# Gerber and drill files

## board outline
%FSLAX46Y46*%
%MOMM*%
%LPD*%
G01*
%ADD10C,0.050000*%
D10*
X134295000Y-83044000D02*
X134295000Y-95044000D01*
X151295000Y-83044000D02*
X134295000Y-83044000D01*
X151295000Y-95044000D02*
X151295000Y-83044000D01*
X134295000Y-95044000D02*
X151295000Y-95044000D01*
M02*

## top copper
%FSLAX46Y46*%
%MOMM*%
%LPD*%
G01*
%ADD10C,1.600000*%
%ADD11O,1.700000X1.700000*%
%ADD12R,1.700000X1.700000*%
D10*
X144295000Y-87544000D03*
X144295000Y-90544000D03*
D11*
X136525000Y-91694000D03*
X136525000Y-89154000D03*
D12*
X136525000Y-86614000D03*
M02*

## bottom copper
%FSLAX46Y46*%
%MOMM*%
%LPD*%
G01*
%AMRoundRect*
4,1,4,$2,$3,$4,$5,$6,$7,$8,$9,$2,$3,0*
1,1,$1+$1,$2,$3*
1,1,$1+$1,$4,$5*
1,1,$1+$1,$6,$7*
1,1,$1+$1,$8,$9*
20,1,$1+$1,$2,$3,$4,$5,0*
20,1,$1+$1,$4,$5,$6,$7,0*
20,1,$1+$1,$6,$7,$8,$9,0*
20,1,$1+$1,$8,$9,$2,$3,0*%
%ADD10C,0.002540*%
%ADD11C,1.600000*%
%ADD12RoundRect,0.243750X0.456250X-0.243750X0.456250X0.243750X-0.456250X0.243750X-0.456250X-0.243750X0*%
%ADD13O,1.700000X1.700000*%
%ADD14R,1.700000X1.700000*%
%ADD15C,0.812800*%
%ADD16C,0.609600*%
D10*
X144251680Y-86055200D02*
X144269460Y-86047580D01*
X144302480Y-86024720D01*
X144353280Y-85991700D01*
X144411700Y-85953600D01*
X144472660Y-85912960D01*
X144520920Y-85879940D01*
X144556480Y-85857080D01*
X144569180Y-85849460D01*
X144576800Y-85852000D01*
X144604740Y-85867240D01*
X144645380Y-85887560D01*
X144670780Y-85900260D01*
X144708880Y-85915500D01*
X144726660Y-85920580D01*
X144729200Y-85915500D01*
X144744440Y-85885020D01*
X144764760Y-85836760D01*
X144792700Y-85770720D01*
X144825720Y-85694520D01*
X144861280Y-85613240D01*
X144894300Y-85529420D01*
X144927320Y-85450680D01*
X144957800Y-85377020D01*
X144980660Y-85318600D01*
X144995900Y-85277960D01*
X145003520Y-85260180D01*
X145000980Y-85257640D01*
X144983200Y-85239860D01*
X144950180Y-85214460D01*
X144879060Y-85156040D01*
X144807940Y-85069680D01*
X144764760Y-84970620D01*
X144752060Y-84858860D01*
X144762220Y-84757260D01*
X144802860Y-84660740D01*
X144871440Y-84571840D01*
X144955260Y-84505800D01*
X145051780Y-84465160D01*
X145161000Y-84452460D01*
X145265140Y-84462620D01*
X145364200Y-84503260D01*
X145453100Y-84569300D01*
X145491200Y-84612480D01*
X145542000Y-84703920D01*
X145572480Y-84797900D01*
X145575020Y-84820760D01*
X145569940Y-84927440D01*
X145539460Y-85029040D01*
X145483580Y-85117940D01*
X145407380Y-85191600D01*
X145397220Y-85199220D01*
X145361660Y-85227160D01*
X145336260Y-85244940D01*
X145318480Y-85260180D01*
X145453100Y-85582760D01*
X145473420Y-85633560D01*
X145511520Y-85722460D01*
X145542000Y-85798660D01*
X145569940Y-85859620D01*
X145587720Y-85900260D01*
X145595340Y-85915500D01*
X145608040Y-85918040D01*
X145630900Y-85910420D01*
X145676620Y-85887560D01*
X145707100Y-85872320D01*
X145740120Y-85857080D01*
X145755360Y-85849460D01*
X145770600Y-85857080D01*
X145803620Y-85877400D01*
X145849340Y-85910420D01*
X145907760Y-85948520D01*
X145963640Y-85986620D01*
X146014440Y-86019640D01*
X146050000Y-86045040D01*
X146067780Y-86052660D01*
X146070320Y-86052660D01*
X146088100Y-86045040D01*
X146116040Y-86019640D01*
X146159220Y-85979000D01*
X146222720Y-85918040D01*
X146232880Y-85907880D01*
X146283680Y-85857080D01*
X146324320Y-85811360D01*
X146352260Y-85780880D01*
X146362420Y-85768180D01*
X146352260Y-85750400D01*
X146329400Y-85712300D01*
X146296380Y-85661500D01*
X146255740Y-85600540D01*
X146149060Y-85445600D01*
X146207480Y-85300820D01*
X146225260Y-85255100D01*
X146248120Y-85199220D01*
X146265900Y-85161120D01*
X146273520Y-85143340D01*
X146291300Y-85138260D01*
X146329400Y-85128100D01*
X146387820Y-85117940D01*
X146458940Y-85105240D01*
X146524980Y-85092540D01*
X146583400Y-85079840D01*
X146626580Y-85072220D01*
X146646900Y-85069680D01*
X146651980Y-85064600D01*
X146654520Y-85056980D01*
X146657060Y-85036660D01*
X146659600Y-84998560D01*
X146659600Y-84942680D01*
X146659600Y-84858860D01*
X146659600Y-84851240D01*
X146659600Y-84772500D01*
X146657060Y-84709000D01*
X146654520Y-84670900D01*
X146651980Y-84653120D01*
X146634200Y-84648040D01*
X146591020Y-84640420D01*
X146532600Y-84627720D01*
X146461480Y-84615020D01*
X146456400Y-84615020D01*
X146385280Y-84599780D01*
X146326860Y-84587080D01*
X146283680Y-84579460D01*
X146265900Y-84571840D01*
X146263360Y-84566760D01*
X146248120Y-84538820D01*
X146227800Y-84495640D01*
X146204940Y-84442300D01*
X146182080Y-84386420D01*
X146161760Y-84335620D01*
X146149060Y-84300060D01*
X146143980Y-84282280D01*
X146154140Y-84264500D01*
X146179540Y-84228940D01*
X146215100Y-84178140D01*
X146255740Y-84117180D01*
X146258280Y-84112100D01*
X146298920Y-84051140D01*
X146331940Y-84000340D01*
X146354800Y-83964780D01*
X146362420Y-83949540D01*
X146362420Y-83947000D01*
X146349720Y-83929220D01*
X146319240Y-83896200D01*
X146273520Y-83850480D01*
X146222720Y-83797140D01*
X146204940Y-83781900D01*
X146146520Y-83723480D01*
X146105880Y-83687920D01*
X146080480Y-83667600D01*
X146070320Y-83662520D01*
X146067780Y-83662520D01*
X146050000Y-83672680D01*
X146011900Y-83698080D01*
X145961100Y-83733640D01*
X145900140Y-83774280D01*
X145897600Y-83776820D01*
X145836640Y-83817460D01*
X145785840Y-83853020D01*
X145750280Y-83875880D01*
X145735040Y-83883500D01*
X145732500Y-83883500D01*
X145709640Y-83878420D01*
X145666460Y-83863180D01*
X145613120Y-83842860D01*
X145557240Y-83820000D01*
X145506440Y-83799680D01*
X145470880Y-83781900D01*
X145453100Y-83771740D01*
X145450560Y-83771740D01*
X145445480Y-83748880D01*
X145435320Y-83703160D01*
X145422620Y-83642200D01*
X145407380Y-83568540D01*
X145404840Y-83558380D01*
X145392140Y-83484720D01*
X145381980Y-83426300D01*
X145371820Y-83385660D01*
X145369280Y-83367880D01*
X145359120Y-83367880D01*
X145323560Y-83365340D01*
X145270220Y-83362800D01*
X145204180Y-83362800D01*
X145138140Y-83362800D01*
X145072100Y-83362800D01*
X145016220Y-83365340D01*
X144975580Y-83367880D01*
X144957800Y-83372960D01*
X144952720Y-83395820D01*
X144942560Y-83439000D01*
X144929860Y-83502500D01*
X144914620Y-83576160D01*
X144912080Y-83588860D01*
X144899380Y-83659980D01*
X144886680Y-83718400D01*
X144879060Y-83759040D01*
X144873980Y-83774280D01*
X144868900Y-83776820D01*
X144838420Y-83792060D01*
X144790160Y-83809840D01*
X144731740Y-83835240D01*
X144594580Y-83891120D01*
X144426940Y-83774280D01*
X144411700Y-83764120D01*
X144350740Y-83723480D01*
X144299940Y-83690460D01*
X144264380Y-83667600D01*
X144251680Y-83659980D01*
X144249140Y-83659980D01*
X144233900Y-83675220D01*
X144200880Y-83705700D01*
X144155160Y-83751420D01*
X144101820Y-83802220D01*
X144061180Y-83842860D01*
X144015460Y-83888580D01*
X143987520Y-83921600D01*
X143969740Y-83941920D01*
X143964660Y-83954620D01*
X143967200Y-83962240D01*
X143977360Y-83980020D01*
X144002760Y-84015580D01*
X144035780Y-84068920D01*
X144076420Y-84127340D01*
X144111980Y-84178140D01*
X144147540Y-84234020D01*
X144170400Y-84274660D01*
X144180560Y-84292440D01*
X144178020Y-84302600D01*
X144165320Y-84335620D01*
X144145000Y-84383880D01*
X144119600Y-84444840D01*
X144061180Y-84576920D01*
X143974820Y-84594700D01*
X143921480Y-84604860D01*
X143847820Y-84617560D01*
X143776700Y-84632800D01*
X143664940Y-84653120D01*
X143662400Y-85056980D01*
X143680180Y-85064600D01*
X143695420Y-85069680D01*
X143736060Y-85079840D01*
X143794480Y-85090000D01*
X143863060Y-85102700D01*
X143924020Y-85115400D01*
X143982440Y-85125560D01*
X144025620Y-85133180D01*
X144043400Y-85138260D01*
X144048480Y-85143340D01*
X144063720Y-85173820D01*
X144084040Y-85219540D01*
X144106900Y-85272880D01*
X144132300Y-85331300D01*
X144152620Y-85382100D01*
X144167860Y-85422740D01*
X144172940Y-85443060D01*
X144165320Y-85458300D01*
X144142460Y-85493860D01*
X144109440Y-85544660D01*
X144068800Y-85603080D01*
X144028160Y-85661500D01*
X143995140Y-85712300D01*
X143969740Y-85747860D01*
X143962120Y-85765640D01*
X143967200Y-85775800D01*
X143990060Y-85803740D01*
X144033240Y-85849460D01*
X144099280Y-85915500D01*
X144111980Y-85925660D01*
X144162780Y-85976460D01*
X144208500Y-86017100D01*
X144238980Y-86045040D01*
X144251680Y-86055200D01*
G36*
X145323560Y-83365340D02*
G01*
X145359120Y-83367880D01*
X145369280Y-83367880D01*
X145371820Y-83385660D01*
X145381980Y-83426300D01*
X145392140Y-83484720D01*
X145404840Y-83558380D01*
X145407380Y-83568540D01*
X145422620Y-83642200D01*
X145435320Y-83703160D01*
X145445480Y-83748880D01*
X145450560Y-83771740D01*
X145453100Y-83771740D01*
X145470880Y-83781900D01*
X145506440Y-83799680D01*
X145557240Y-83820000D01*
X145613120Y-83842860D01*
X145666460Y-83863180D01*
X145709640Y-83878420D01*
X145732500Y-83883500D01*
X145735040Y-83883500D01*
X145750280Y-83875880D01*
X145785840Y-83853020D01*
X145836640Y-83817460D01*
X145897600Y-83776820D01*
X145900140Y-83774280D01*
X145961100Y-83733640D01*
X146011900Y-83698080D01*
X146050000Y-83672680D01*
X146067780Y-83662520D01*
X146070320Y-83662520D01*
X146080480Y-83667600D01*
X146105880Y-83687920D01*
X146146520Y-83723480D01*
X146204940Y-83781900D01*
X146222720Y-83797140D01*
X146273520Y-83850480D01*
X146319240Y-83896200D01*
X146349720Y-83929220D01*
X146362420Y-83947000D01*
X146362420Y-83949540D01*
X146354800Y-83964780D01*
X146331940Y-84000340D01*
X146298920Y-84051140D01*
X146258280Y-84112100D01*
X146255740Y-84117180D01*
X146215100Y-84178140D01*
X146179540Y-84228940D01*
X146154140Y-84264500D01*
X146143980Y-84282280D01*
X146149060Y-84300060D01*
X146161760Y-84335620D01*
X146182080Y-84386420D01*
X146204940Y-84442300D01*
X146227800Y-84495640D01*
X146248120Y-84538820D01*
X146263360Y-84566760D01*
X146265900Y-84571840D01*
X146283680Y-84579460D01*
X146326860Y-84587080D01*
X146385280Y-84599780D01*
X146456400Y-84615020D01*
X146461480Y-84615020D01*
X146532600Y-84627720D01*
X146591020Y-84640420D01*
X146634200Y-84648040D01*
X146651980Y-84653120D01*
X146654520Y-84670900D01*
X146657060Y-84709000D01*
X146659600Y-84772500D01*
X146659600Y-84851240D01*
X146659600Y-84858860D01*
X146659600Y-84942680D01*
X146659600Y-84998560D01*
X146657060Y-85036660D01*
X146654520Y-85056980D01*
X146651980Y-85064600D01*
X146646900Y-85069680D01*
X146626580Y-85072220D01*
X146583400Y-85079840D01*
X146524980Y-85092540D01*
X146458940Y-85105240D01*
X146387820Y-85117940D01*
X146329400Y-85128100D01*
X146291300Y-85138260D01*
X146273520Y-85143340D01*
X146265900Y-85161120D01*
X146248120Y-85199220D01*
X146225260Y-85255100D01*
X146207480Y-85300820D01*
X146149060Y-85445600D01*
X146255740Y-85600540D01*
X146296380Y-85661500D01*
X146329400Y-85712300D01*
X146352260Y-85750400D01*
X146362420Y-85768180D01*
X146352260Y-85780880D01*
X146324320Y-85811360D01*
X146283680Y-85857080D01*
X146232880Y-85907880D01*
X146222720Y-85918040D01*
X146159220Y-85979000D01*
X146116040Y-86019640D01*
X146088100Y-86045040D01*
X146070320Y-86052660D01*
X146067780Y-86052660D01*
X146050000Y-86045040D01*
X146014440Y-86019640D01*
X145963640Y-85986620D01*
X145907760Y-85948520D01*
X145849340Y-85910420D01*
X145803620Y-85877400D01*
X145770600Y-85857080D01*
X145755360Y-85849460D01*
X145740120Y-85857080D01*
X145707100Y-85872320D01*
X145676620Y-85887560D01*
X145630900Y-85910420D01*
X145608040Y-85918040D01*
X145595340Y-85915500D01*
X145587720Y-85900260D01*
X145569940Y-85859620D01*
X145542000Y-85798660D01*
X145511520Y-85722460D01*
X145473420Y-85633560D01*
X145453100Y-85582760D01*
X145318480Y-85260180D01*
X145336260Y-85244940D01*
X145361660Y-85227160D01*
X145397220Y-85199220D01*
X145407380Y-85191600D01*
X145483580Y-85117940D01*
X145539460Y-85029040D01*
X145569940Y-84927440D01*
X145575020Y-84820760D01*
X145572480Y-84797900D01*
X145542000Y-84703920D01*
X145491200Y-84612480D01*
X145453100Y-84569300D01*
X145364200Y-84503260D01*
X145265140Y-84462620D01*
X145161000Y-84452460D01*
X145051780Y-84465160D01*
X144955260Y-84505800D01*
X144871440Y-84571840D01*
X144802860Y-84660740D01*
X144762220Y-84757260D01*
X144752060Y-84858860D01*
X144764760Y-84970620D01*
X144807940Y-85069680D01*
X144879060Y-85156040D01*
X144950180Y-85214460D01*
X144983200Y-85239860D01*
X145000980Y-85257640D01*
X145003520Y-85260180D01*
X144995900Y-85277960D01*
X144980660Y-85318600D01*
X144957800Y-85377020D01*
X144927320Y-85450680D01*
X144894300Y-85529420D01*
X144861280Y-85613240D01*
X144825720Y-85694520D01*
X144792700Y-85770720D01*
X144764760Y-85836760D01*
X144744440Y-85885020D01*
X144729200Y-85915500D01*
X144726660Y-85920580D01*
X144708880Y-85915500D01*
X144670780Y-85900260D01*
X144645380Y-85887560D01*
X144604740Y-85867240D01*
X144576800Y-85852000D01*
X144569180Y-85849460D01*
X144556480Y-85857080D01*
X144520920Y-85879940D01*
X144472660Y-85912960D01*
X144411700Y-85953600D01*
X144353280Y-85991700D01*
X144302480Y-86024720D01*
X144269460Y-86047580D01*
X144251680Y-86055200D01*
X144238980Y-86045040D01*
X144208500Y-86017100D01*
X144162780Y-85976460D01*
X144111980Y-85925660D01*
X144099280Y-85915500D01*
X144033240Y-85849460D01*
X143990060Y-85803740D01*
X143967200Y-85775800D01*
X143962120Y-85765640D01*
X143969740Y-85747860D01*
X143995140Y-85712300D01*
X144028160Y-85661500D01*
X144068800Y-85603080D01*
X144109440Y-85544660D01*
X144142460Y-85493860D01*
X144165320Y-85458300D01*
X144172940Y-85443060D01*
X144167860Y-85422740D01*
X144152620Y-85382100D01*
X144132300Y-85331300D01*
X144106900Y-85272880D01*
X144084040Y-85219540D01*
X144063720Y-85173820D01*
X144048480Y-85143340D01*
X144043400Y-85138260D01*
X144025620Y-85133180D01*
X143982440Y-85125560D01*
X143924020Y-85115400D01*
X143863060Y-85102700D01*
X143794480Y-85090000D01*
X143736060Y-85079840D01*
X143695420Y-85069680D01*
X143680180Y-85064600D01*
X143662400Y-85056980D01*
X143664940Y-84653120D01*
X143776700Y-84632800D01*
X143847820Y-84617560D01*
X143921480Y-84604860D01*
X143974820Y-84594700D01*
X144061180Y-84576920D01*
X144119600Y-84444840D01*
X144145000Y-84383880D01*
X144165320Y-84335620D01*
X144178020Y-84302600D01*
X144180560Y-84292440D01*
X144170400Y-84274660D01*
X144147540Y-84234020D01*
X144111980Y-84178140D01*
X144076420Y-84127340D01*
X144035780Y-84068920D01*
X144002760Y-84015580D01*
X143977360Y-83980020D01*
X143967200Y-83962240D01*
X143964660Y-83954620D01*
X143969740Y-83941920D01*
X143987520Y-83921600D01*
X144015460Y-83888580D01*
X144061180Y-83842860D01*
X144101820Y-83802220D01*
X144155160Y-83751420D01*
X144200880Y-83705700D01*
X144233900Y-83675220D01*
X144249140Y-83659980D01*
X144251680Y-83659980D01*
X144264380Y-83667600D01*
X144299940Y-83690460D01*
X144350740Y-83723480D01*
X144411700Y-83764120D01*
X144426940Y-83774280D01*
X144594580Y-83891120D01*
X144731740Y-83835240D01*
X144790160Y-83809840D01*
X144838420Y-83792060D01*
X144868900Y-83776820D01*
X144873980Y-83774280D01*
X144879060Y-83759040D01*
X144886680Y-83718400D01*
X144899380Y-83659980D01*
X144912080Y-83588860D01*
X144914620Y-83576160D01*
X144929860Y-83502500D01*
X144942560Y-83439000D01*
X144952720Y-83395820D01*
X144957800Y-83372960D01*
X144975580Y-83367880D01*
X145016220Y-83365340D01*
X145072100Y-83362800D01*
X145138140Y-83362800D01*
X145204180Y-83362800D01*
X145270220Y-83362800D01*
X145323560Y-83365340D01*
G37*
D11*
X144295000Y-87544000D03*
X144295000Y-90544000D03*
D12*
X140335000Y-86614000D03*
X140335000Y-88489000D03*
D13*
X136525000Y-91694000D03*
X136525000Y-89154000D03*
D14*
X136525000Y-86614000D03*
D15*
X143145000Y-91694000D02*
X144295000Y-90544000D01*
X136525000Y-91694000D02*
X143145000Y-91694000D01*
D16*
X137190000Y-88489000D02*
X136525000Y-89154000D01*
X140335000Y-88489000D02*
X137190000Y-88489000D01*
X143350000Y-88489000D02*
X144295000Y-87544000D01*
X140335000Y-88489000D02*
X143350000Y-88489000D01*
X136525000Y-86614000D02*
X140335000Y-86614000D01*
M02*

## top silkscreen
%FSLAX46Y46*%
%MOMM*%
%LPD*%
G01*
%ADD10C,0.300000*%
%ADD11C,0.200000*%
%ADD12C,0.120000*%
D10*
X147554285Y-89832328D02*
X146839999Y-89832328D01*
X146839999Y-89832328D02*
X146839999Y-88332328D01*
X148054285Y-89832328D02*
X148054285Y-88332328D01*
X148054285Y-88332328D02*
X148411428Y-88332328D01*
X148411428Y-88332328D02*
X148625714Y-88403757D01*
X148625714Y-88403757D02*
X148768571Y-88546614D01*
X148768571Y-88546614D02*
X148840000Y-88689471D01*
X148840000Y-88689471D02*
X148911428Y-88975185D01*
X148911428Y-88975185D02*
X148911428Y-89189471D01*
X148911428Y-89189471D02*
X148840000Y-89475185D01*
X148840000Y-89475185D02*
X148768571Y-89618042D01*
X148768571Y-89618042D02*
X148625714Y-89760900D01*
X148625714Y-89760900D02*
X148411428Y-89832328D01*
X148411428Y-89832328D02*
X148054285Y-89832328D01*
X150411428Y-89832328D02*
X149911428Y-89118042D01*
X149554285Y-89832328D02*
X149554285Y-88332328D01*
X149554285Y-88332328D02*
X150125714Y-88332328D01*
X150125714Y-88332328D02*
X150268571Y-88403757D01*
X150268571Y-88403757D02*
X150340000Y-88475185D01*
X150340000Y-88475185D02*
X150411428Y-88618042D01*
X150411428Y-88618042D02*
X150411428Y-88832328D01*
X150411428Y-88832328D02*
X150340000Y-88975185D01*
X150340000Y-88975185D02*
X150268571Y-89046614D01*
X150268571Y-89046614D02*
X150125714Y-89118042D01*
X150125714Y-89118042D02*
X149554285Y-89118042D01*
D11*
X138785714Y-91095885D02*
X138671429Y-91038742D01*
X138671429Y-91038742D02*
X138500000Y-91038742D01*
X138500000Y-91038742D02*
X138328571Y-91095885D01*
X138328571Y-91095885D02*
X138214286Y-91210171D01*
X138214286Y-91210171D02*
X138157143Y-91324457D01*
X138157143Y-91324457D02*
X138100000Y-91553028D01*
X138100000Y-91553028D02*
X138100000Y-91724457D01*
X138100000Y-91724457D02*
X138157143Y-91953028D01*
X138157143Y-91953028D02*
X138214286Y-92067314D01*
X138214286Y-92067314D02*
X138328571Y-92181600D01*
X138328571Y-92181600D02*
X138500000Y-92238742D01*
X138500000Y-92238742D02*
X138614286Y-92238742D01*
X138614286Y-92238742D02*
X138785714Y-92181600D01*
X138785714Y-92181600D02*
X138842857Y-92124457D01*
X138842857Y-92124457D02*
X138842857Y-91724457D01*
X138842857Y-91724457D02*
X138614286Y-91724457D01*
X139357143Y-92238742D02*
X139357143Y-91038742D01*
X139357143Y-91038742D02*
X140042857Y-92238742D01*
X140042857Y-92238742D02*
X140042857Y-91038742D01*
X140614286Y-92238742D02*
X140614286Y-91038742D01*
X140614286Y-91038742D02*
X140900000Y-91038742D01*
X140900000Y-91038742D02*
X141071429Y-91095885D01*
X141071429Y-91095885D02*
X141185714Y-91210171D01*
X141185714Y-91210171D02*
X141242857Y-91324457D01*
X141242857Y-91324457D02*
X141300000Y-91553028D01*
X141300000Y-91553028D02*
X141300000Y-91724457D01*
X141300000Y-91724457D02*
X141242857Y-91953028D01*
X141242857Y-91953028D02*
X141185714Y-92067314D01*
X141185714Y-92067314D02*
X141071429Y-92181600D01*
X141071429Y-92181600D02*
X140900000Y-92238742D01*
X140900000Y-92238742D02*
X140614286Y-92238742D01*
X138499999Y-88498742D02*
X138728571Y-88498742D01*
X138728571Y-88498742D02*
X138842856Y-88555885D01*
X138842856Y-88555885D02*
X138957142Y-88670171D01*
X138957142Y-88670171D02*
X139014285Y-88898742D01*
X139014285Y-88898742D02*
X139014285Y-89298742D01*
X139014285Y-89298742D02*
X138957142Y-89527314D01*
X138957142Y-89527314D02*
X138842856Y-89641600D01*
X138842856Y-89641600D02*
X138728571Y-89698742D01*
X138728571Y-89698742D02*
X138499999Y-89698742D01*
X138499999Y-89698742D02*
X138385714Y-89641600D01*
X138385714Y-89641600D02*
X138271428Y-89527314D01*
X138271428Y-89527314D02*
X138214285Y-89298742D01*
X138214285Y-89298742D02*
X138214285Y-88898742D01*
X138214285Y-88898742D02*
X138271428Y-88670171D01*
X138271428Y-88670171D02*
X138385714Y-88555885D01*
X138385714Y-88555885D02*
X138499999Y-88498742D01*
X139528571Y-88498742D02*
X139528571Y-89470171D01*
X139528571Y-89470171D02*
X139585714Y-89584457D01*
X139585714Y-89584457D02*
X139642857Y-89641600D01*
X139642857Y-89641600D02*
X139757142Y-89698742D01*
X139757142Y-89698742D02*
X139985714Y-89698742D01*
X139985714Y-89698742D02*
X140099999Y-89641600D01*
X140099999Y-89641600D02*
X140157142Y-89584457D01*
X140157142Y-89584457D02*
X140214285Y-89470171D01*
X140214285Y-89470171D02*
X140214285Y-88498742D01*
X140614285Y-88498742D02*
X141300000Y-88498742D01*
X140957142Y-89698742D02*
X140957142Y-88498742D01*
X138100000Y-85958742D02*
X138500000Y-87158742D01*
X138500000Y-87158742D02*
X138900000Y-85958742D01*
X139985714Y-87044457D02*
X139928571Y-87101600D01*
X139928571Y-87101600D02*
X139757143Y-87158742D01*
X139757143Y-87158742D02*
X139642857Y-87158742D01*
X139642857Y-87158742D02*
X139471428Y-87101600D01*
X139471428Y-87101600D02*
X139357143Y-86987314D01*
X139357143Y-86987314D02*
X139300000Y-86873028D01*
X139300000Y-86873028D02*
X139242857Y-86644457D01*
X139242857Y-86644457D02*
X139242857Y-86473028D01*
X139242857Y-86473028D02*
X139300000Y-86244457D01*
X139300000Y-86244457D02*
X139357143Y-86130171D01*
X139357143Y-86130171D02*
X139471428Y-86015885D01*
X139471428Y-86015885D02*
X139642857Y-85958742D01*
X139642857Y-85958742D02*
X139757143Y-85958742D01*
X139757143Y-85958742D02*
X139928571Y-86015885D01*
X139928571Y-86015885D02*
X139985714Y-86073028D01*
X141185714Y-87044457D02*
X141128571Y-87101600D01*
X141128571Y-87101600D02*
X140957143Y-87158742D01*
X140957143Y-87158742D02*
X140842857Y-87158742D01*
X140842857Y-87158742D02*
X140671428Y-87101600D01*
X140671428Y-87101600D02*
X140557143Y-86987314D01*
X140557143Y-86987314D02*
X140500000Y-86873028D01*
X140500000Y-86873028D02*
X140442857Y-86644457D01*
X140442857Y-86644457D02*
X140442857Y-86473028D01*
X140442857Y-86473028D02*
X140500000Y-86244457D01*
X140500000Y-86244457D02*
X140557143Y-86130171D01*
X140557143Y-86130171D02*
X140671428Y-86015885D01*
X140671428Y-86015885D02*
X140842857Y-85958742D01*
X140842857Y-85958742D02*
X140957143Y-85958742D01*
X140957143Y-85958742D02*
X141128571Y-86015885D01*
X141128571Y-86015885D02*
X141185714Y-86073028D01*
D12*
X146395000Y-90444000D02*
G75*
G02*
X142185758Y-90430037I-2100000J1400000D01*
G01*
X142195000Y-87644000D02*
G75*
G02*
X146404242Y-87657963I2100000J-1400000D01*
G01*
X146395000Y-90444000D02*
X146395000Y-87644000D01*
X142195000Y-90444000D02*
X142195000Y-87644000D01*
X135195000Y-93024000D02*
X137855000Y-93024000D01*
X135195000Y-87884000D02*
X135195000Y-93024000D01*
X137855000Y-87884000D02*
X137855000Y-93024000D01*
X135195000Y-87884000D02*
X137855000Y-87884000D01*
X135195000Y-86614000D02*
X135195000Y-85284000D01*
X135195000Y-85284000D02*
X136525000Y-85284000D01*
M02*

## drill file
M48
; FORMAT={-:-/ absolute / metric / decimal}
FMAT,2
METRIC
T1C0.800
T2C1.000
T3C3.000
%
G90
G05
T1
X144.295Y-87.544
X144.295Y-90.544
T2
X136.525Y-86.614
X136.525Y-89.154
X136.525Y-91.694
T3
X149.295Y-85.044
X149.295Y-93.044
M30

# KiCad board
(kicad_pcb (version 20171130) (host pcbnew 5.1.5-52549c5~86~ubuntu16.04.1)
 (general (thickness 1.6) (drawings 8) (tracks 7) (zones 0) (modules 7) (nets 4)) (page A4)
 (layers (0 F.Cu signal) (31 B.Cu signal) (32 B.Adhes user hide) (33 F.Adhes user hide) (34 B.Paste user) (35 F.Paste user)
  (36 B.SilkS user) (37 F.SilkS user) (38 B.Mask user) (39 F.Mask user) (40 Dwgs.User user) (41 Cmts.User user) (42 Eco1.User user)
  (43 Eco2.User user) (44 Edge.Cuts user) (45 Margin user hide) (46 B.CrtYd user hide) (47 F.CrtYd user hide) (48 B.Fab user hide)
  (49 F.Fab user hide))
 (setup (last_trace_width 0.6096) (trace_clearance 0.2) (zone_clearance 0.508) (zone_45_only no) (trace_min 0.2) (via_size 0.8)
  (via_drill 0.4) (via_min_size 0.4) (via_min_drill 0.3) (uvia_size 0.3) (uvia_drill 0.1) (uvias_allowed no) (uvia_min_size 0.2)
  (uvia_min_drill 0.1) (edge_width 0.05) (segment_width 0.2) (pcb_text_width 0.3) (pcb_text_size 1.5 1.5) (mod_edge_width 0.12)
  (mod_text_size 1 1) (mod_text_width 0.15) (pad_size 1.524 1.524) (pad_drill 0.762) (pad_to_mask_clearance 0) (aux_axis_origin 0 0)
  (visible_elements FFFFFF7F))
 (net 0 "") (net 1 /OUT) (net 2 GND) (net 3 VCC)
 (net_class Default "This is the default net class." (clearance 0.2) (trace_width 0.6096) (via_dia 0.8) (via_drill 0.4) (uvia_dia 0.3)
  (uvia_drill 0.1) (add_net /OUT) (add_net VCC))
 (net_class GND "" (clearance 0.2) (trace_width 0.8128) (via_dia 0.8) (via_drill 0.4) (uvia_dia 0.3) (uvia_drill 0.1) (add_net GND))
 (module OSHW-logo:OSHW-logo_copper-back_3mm (layer B.Cu) (at 145.161 84.709 180)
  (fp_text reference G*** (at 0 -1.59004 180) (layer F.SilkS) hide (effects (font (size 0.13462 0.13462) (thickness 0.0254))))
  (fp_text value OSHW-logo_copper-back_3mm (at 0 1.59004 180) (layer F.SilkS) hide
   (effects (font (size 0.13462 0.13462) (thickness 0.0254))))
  (fp_poly
   (pts (xy 0.90932 -1.3462) (xy 0.89154 -1.33858) (xy 0.85852 -1.31572) (xy 0.80772 -1.2827) (xy 0.7493 -1.2446) (xy 0.68834 -1.20396)
    (xy 0.64008 -1.17094) (xy 0.60452 -1.14808) (xy 0.59182 -1.14046) (xy 0.5842 -1.143) (xy 0.55626 -1.15824) (xy 0.51562 -1.17856)
    (xy 0.49022 -1.19126) (xy 0.45212 -1.2065) (xy 0.43434 -1.21158) (xy 0.4318 -1.2065) (xy 0.41656 -1.17602) (xy 0.39624 -1.12776)
    (xy 0.3683 -1.06172) (xy 0.33528 -0.98552) (xy 0.29972 -0.90424) (xy 0.2667 -0.82042) (xy 0.23368 -0.74168) (xy 0.2032 -0.66802)
    (xy 0.18034 -0.6096) (xy 0.1651 -0.56896) (xy 0.15748 -0.55118) (xy 0.16002 -0.54864) (xy 0.1778 -0.53086) (xy 0.21082 -0.50546)
    (xy 0.28194 -0.44704) (xy 0.35306 -0.36068) (xy 0.39624 -0.26162) (xy 0.40894 -0.14986) (xy 0.39878 -0.04826) (xy 0.35814 0.04826)
    (xy 0.28956 0.13716) (xy 0.20574 0.2032) (xy 0.10922 0.24384) (xy 0 0.25654) (xy -0.10414 0.24638) (xy -0.2032 0.20574)
    (xy -0.2921 0.1397) (xy -0.3302 0.09652) (xy -0.381 0.00508) (xy -0.41148 -0.0889) (xy -0.41402 -0.11176) (xy -0.40894 -0.21844)
    (xy -0.37846 -0.32004) (xy -0.32258 -0.40894) (xy -0.24638 -0.4826) (xy -0.23622 -0.49022) (xy -0.20066 -0.51816) (xy -0.17526 -0.53594)
    (xy -0.15748 -0.55118) (xy -0.2921 -0.87376) (xy -0.31242 -0.92456) (xy -0.35052 -1.01346) (xy -0.381 -1.08966) (xy -0.40894 -1.15062)
    (xy -0.42672 -1.19126) (xy -0.43434 -1.2065) (xy -0.44704 -1.20904) (xy -0.4699 -1.20142) (xy -0.51562 -1.17856) (xy -0.5461 -1.16332)
    (xy -0.57912 -1.14808) (xy -0.59436 -1.14046) (xy -0.6096 -1.14808) (xy -0.64262 -1.1684) (xy -0.68834 -1.20142) (xy -0.74676 -1.23952)
    (xy -0.80264 -1.27762) (xy -0.85344 -1.31064) (xy -0.889 -1.33604) (xy -0.90678 -1.34366) (xy -0.90932 -1.34366) (xy -0.9271 -1.33604)
    (xy -0.95504 -1.31064) (xy -0.99822 -1.27) (xy -1.06172 -1.20904) (xy -1.07188 -1.19888) (xy -1.12268 -1.14808) (xy -1.16332 -1.10236)
    (xy -1.19126 -1.07188) (xy -1.20142 -1.05918) (xy -1.19126 -1.0414) (xy -1.1684 -1.0033) (xy -1.13538 -0.9525) (xy -1.09474 -0.89154)
    (xy -0.98806 -0.7366) (xy -1.04648 -0.59182) (xy -1.06426 -0.5461) (xy -1.08712 -0.49022) (xy -1.1049 -0.45212) (xy -1.11252 -0.43434)
    (xy -1.1303 -0.42926) (xy -1.1684 -0.4191) (xy -1.22682 -0.40894) (xy -1.29794 -0.39624) (xy -1.36398 -0.38354) (xy -1.4224 -0.37084)
    (xy -1.46558 -0.36322) (xy -1.4859 -0.36068) (xy -1.49098 -0.3556) (xy -1.49352 -0.34798) (xy -1.49606 -0.32766) (xy -1.4986 -0.28956)
    (xy -1.4986 -0.23368) (xy -1.4986 -0.14986) (xy -1.4986 -0.14224) (xy -1.4986 -0.0635) (xy -1.49606 0) (xy -1.49352 0.0381)
    (xy -1.49098 0.05588) (xy -1.4732 0.06096) (xy -1.43002 0.06858) (xy -1.3716 0.08128) (xy -1.30048 0.09398) (xy -1.2954 0.09398)
    (xy -1.22428 0.10922) (xy -1.16586 0.12192) (xy -1.12268 0.12954) (xy -1.1049 0.13716) (xy -1.10236 0.14224) (xy -1.08712 0.17018)
    (xy -1.0668 0.21336) (xy -1.04394 0.2667) (xy -1.02108 0.32258) (xy -1.00076 0.37338) (xy -0.98806 0.40894) (xy -0.98298 0.42672)
    (xy -0.99314 0.4445) (xy -1.01854 0.48006) (xy -1.0541 0.53086) (xy -1.09474 0.59182) (xy -1.09728 0.5969) (xy -1.13792 0.65786)
    (xy -1.17094 0.70866) (xy -1.1938 0.74422) (xy -1.20142 0.75946) (xy -1.20142 0.762) (xy -1.18872 0.77978) (xy -1.15824 0.8128)
    (xy -1.11252 0.85852) (xy -1.06172 0.91186) (xy -1.04394 0.9271) (xy -0.98552 0.98552) (xy -0.94488 1.02108) (xy -0.91948 1.0414)
    (xy -0.90932 1.04648) (xy -0.90678 1.04648) (xy -0.889 1.03632) (xy -0.8509 1.01092) (xy -0.8001 0.97536) (xy -0.73914 0.93472)
    (xy -0.7366 0.93218) (xy -0.67564 0.89154) (xy -0.62484 0.85598) (xy -0.58928 0.83312) (xy -0.57404 0.8255) (xy -0.5715 0.8255)
    (xy -0.54864 0.83058) (xy -0.50546 0.84582) (xy -0.45212 0.86614) (xy -0.39624 0.889) (xy -0.34544 0.90932) (xy -0.30988 0.9271)
    (xy -0.2921 0.93726) (xy -0.28956 0.93726) (xy -0.28448 0.96012) (xy -0.27432 1.00584) (xy -0.26162 1.0668) (xy -0.24638 1.14046)
    (xy -0.24384 1.15062) (xy -0.23114 1.22428) (xy -0.22098 1.2827) (xy -0.21082 1.32334) (xy -0.20828 1.34112) (xy -0.19812 1.34112)
    (xy -0.16256 1.34366) (xy -0.10922 1.3462) (xy -0.04318 1.3462) (xy 0.02286 1.3462) (xy 0.0889 1.3462) (xy 0.14478 1.34366)
    (xy 0.18542 1.34112) (xy 0.2032 1.33604) (xy 0.20828 1.31318) (xy 0.21844 1.27) (xy 0.23114 1.2065) (xy 0.24638 1.13284)
    (xy 0.24892 1.12014) (xy 0.26162 1.04902) (xy 0.27432 0.9906) (xy 0.28194 0.94996) (xy 0.28702 0.93472) (xy 0.2921 0.93218)
    (xy 0.32258 0.91694) (xy 0.37084 0.89916) (xy 0.42926 0.87376) (xy 0.56642 0.81788) (xy 0.73406 0.93472) (xy 0.7493 0.94488)
    (xy 0.81026 0.98552) (xy 0.86106 1.01854) (xy 0.89662 1.0414) (xy 0.90932 1.04902) (xy 0.91186 1.04902) (xy 0.9271 1.03378)
    (xy 0.96012 1.0033) (xy 1.00584 0.95758) (xy 1.05918 0.90678) (xy 1.09982 0.86614) (xy 1.14554 0.82042) (xy 1.17348 0.7874)
    (xy 1.19126 0.76708) (xy 1.19634 0.75438) (xy 1.1938 0.74676) (xy 1.18364 0.72898) (xy 1.15824 0.69342) (xy 1.12522 0.64008)
    (xy 1.08458 0.58166) (xy 1.04902 0.53086) (xy 1.01346 0.47498) (xy 0.9906 0.43434) (xy 0.98044 0.41656) (xy 0.98298 0.4064)
    (xy 0.99568 0.37338) (xy 1.016 0.32512) (xy 1.0414 0.26416) (xy 1.09982 0.13208) (xy 1.18618 0.1143) (xy 1.23952 0.10414)
    (xy 1.31318 0.09144) (xy 1.3843 0.0762) (xy 1.49606 0.05588) (xy 1.4986 -0.34798) (xy 1.48082 -0.3556) (xy 1.46558 -0.36068)
    (xy 1.42494 -0.37084) (xy 1.36652 -0.381) (xy 1.29794 -0.3937) (xy 1.23698 -0.4064) (xy 1.17856 -0.41656) (xy 1.13538 -0.42418)
    (xy 1.1176 -0.42926) (xy 1.11252 -0.43434) (xy 1.09728 -0.46482) (xy 1.07696 -0.51054) (xy 1.0541 -0.56388) (xy 1.0287 -0.6223)
    (xy 1.00838 -0.6731) (xy 0.99314 -0.71374) (xy 0.98806 -0.73406) (xy 0.99568 -0.7493) (xy 1.01854 -0.78486) (xy 1.05156 -0.83566)
    (xy 1.0922 -0.89408) (xy 1.13284 -0.9525) (xy 1.16586 -1.0033) (xy 1.19126 -1.03886) (xy 1.19888 -1.05664) (xy 1.1938 -1.0668)
    (xy 1.17094 -1.09474) (xy 1.12776 -1.14046) (xy 1.06172 -1.2065) (xy 1.04902 -1.21666) (xy 0.99822 -1.26746) (xy 0.9525 -1.3081)
    (xy 0.92202 -1.33604) (xy 0.90932 -1.3462))
   (layer B.Cu) (width 0.00254)))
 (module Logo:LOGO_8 (layer B.Cu) (at 142.881524 93.322196 180)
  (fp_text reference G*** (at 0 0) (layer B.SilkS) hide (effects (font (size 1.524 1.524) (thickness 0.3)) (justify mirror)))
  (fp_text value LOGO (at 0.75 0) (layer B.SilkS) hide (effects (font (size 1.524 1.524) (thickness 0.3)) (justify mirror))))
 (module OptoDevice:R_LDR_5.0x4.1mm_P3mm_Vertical (layer F.Cu) (at 144.295 90.544 90)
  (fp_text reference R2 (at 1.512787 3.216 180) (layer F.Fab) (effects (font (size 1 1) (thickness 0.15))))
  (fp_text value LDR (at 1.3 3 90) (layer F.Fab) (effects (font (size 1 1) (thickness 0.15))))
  (fp_arc (start 1.5 0) (end 0.1 2.1) (angle 113) (layer F.SilkS) (width 0.12))
  (fp_arc (start 1.5 0) (end 2.9 -2.1) (angle 113) (layer F.SilkS) (width 0.12))
  (fp_line (start 0.1 2.1) (end 2.9 2.1) (layer F.SilkS) (width 0.12))
  (fp_line (start 0.1 -2.1) (end 2.9 -2.1) (layer F.SilkS) (width 0.12))
  (pad 2 thru_hole circle (at 3 0 90) (size 1.6 1.6) (drill 0.8) (layers *.Cu *.Mask) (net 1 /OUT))
  (pad 1 thru_hole circle (at 0 0 90) (size 1.6 1.6) (drill 0.8) (layers *.Cu *.Mask) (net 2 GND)))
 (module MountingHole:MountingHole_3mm (layer F.Cu) (at 149.295 85.044)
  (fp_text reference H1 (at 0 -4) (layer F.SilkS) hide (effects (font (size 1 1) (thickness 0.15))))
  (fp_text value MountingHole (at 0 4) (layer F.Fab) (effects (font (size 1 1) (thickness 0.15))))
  (pad 1 np_thru_hole circle (at 0 0) (size 3 3) (drill 3) (layers *.Cu *.Mask)))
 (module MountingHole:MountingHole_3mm (layer F.Cu) (at 149.295 93.044)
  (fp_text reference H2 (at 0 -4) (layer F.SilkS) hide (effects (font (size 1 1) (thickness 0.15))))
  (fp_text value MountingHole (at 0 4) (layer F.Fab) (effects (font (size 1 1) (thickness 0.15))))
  (pad 1 np_thru_hole circle (at 0 0) (size 3 3) (drill 3) (layers *.Cu *.Mask)))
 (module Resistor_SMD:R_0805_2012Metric (layer B.Cu) (at 140.335 87.5515 90)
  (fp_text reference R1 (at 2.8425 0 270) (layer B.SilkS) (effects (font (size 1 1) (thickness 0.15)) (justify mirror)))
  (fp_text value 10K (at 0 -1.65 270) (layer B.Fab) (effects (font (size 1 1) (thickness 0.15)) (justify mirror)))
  (pad 2 smd roundrect (at 0.9375 0 90) (size 0.975 1.4) (layers B.Cu B.Paste B.Mask) (roundrect_rratio 0.25) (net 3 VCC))
  (pad 1 smd roundrect (at -0.9375 0 90) (size 0.975 1.4) (layers B.Cu B.Paste B.Mask) (roundrect_rratio 0.25) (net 1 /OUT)))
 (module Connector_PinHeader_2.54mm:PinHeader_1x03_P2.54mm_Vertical (layer F.Cu) (at 136.525 86.614)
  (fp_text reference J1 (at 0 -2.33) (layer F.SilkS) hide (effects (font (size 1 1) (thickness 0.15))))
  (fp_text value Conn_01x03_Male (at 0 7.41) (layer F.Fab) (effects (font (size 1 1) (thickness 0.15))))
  (fp_line (start -1.33 6.41) (end 1.33 6.41) (layer F.SilkS) (width 0.12))
  (fp_line (start -1.33 1.27) (end -1.33 6.41) (layer F.SilkS) (width 0.12))
  (fp_line (start 1.33 1.27) (end 1.33 6.41) (layer F.SilkS) (width 0.12))
  (fp_line (start -1.33 1.27) (end 1.33 1.27) (layer F.SilkS) (width 0.12))
  (fp_line (start -1.33 0) (end -1.33 -1.33) (layer F.SilkS) (width 0.12))
  (fp_line (start -1.33 -1.33) (end 0 -1.33) (layer F.SilkS) (width 0.12))
  (pad 3 thru_hole oval (at 0 5.08) (size 1.7 1.7) (drill 1) (layers *.Cu *.Mask) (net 2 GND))
  (pad 2 thru_hole oval (at 0 2.54) (size 1.7 1.7) (drill 1) (layers *.Cu *.Mask) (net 1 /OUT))
  (pad 1 thru_hole rect (at 0 0) (size 1.7 1.7) (drill 1) (layers *.Cu *.Mask) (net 3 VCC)))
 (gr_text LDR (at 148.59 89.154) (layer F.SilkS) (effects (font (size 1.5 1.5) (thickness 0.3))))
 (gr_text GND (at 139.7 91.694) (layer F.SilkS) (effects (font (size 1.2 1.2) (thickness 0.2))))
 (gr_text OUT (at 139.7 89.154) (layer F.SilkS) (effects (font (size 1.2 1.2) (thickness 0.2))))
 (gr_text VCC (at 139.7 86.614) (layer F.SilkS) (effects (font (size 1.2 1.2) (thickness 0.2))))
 (gr_line (start 134.295 83.044) (end 134.295 95.044) (layer Edge.Cuts) (width 0.05))
 (gr_line (start 151.295 83.044) (end 134.295 83.044) (layer Edge.Cuts) (width 0.05))
 (gr_line (start 151.295 95.044) (end 151.295 83.044) (layer Edge.Cuts) (width 0.05))
 (gr_line (start 134.295 95.044) (end 151.295 95.044) (layer Edge.Cuts) (width 0.05))
 (segment (start 143.145 91.694) (end 144.295 90.544) (width 0.8128) (layer B.Cu) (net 2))
 (segment (start 136.525 91.694) (end 143.145 91.694) (width 0.8128) (layer B.Cu) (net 2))
 (segment (start 137.19 88.489) (end 136.525 89.154) (width 0.6096) (layer B.Cu) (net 1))
 (segment (start 140.335 88.489) (end 137.19 88.489) (width 0.6096) (layer B.Cu) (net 1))
 (segment (start 143.35 88.489) (end 144.295 87.544) (width 0.6096) (layer B.Cu) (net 1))
 (segment (start 140.335 88.489) (end 143.35 88.489) (width 0.6096) (layer B.Cu) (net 1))
 (segment (start 136.525 86.614) (end 140.335 86.614) (width 0.6096) (layer B.Cu) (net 3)))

